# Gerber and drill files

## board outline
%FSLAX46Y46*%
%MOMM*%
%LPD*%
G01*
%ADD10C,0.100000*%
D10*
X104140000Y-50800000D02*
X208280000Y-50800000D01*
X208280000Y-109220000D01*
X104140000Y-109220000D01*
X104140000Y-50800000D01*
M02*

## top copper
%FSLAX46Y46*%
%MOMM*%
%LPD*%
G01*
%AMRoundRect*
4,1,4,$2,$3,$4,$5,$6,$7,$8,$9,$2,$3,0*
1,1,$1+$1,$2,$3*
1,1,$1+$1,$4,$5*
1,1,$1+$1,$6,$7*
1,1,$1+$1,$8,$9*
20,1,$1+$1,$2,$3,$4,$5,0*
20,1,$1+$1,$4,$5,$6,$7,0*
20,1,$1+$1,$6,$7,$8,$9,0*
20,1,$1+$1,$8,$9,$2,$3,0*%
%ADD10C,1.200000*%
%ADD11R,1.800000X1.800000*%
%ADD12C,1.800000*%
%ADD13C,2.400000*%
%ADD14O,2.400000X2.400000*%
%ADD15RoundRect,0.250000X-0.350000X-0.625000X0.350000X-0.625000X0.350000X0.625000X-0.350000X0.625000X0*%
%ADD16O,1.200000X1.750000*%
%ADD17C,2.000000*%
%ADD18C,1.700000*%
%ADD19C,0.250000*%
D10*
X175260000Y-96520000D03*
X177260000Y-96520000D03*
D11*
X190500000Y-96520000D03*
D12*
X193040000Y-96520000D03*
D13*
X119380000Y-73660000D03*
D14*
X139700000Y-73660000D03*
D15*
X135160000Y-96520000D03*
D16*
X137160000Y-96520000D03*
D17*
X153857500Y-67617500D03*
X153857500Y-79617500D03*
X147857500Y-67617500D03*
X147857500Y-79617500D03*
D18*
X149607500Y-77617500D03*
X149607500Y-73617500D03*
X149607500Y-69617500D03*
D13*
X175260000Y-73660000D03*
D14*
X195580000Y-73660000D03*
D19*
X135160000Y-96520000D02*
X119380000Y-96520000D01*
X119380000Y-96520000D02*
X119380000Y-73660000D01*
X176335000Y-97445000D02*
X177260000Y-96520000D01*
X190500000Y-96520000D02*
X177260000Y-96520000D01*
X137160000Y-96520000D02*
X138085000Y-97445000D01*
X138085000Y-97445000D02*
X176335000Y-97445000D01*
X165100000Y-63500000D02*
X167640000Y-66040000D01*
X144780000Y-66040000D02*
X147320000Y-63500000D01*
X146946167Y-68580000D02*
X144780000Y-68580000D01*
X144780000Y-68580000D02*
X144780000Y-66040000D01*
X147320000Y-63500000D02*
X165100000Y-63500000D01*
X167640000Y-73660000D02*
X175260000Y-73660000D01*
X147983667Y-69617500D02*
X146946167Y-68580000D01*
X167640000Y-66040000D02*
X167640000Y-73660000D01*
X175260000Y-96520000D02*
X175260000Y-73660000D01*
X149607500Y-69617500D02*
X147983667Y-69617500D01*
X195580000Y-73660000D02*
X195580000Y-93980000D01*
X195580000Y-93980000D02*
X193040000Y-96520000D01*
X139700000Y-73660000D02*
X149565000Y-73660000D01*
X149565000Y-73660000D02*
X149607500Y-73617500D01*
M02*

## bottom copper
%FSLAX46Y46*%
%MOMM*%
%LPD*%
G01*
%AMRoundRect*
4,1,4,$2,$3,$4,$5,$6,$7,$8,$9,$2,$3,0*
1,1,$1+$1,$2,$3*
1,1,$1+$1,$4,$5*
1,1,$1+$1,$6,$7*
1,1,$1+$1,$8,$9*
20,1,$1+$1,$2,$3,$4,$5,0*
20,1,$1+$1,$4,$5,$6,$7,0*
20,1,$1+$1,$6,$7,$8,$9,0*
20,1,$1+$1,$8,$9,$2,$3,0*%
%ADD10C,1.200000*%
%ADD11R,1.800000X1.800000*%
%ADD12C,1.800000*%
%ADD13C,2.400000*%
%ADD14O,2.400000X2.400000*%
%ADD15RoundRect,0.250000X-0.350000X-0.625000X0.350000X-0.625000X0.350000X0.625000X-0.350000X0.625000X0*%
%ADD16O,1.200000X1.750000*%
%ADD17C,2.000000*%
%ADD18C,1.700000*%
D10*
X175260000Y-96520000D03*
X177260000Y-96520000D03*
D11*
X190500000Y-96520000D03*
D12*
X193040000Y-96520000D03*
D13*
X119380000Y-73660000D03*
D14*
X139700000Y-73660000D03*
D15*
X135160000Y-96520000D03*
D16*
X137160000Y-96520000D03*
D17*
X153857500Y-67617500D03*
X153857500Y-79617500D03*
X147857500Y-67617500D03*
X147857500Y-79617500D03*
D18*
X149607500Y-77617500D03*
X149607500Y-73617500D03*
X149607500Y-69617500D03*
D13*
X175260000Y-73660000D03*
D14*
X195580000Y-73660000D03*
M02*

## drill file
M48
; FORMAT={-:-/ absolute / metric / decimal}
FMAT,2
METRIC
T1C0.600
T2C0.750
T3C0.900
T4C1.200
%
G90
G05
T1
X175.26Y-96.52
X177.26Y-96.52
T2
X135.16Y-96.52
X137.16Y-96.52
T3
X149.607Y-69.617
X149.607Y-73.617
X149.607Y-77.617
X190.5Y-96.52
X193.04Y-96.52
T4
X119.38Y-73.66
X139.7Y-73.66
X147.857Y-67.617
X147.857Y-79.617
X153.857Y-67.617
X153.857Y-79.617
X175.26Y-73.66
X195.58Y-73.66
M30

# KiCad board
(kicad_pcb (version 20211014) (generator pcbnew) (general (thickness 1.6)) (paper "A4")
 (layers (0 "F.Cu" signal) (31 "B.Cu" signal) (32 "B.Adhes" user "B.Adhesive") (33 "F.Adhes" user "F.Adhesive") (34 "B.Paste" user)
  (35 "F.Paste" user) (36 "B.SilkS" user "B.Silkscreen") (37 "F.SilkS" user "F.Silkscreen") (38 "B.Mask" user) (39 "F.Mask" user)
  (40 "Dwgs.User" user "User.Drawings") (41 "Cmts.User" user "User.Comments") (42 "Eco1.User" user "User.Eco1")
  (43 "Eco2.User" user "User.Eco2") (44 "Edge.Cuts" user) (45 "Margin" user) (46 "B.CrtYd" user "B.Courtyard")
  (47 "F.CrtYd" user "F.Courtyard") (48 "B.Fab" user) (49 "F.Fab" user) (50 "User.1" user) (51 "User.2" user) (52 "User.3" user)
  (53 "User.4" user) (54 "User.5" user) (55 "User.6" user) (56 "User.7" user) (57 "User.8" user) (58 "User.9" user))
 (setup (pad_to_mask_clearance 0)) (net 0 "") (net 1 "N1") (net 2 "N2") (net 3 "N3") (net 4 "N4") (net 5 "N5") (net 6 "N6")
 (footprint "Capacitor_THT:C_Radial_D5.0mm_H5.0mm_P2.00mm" (layer "F.Cu") (at 175.26 96.52)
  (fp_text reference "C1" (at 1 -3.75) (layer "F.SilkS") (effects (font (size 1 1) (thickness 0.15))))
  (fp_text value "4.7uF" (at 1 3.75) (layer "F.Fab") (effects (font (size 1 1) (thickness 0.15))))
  (pad "1" thru_hole circle (at 0 0) (size 1.2 1.2) (drill 0.6) (layers *.Cu *.Mask) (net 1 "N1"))
  (pad "2" thru_hole circle (at 2 0) (size 1.2 1.2) (drill 0.6) (layers *.Cu *.Mask) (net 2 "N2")))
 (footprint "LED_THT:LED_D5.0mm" (layer "F.Cu") (at 190.5 96.52)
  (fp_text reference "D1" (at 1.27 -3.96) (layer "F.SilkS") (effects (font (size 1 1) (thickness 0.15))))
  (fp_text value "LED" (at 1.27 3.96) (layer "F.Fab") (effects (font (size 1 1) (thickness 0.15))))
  (pad "1" thru_hole rect (at 0 0) (size 1.8 1.8) (drill 0.9) (layers *.Cu *.Mask) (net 2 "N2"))
  (pad "2" thru_hole circle (at 2.54 0) (size 1.8 1.8) (drill 0.9) (layers *.Cu *.Mask) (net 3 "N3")))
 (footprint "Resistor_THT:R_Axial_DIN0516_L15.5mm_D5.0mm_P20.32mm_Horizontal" (layer "F.Cu") (at 119.38 73.66)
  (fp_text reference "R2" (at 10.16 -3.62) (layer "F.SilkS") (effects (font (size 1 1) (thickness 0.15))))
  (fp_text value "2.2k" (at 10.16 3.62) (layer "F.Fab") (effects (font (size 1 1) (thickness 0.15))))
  (pad "1" thru_hole circle (at 0 0) (size 2.4 2.4) (drill 1.2) (layers *.Cu *.Mask) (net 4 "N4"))
  (pad "2" thru_hole oval (at 20.32 0) (size 2.4 2.4) (drill 1.2) (layers *.Cu *.Mask) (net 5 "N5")))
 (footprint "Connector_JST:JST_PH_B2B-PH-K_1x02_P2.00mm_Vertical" (layer "F.Cu") (at 135.16 96.52)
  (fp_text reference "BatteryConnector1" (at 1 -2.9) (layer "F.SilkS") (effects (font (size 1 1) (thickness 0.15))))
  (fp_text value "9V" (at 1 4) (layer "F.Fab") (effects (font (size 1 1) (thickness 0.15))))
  (pad "1" thru_hole roundrect (at 0 0) (size 1.2 1.75) (drill 0.75) (layers *.Cu *.Mask) (roundrect_rratio 0.208333) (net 4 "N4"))
  (pad "2" thru_hole oval (at 2 0) (size 1.2 1.75) (drill 0.75) (layers *.Cu *.Mask) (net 2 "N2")))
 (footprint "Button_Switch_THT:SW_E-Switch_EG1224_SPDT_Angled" (layer "F.Cu") (at 149.6075 77.6175 90)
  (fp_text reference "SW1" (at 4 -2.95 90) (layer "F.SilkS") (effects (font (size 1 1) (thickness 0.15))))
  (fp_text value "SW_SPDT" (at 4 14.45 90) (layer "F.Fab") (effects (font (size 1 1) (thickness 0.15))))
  (pad "" thru_hole circle (at 10 4.25 90) (size 2 2) (drill 1.2) (layers *.Cu *.Mask))
  (pad "" thru_hole circle (at -2 4.25 90) (size 2 2) (drill 1.2) (layers *.Cu *.Mask))
  (pad "" thru_hole circle (at 10 -1.75 90) (size 2 2) (drill 1.2) (layers *.Cu *.Mask))
  (pad "" thru_hole circle (at -2 -1.75 90) (size 2 2) (drill 1.2) (layers *.Cu *.Mask))
  (pad "1" thru_hole circle (at 0 0 90) (size 1.7 1.7) (drill 0.9) (layers *.Cu *.Mask) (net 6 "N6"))
  (pad "2" thru_hole circle (at 4 0 90) (size 1.7 1.7) (drill 0.9) (layers *.Cu *.Mask) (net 5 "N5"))
  (pad "3" thru_hole circle (at 8 0 90) (size 1.7 1.7) (drill 0.9) (layers *.Cu *.Mask) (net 1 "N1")))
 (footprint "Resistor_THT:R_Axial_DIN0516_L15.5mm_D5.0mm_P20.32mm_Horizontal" (layer "F.Cu") (at 175.26 73.66)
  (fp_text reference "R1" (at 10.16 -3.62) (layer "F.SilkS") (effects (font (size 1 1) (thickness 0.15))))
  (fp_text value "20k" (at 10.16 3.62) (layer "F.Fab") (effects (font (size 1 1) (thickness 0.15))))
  (pad "1" thru_hole circle (at 0 0) (size 2.4 2.4) (drill 1.2) (layers *.Cu *.Mask) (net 1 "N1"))
  (pad "2" thru_hole oval (at 20.32 0) (size 2.4 2.4) (drill 1.2) (layers *.Cu *.Mask) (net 3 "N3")))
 (gr_rect (start 208.28 109.22) (end 104.14 50.8) (layer "Edge.Cuts") (width 0.1) (fill none))
 (segment (start 135.16 96.52) (end 119.38 96.52) (width 0.25) (layer "F.Cu") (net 4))
 (segment (start 119.38 96.52) (end 119.38 73.66) (width 0.25) (layer "F.Cu") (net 4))
 (segment (start 176.335 97.445) (end 177.26 96.52) (width 0.25) (layer "F.Cu") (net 2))
 (segment (start 190.5 96.52) (end 177.26 96.52) (width 0.25) (layer "F.Cu") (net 2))
 (segment (start 137.16 96.52) (end 138.085 97.445) (width 0.25) (layer "F.Cu") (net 2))
 (segment (start 138.085 97.445) (end 176.335 97.445) (width 0.25) (layer "F.Cu") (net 2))
 (segment (start 165.1 63.5) (end 167.64 66.04) (width 0.25) (layer "F.Cu") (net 1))
 (segment (start 144.78 66.04) (end 147.32 63.5) (width 0.25) (layer "F.Cu") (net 1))
 (segment (start 146.946167 68.58) (end 144.78 68.58) (width 0.25) (layer "F.Cu") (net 1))
 (segment (start 144.78 68.58) (end 144.78 66.04) (width 0.25) (layer "F.Cu") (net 1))
 (segment (start 147.32 63.5) (end 165.1 63.5) (width 0.25) (layer "F.Cu") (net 1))
 (segment (start 167.64 73.66) (end 175.26 73.66) (width 0.25) (layer "F.Cu") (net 1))
 (segment (start 147.983667 69.6175) (end 146.946167 68.58) (width 0.25) (layer "F.Cu") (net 1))
 (segment (start 167.64 66.04) (end 167.64 73.66) (width 0.25) (layer "F.Cu") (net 1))
 (segment (start 175.26 96.52) (end 175.26 73.66) (width 0.25) (layer "F.Cu") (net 1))
 (segment (start 149.6075 69.6175) (end 147.983667 69.6175) (width 0.25) (layer "F.Cu") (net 1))
 (segment (start 195.58 73.66) (end 195.58 93.98) (width 0.25) (layer "F.Cu") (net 3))
 (segment (start 195.58 93.98) (end 193.04 96.52) (width 0.25) (layer "F.Cu") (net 3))
 (segment (start 139.7 73.66) (end 149.565 73.66) (width 0.25) (layer "F.Cu") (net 5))
 (segment (start 149.565 73.66) (end 149.6075 73.6175) (width 0.25) (layer "F.Cu") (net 5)))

